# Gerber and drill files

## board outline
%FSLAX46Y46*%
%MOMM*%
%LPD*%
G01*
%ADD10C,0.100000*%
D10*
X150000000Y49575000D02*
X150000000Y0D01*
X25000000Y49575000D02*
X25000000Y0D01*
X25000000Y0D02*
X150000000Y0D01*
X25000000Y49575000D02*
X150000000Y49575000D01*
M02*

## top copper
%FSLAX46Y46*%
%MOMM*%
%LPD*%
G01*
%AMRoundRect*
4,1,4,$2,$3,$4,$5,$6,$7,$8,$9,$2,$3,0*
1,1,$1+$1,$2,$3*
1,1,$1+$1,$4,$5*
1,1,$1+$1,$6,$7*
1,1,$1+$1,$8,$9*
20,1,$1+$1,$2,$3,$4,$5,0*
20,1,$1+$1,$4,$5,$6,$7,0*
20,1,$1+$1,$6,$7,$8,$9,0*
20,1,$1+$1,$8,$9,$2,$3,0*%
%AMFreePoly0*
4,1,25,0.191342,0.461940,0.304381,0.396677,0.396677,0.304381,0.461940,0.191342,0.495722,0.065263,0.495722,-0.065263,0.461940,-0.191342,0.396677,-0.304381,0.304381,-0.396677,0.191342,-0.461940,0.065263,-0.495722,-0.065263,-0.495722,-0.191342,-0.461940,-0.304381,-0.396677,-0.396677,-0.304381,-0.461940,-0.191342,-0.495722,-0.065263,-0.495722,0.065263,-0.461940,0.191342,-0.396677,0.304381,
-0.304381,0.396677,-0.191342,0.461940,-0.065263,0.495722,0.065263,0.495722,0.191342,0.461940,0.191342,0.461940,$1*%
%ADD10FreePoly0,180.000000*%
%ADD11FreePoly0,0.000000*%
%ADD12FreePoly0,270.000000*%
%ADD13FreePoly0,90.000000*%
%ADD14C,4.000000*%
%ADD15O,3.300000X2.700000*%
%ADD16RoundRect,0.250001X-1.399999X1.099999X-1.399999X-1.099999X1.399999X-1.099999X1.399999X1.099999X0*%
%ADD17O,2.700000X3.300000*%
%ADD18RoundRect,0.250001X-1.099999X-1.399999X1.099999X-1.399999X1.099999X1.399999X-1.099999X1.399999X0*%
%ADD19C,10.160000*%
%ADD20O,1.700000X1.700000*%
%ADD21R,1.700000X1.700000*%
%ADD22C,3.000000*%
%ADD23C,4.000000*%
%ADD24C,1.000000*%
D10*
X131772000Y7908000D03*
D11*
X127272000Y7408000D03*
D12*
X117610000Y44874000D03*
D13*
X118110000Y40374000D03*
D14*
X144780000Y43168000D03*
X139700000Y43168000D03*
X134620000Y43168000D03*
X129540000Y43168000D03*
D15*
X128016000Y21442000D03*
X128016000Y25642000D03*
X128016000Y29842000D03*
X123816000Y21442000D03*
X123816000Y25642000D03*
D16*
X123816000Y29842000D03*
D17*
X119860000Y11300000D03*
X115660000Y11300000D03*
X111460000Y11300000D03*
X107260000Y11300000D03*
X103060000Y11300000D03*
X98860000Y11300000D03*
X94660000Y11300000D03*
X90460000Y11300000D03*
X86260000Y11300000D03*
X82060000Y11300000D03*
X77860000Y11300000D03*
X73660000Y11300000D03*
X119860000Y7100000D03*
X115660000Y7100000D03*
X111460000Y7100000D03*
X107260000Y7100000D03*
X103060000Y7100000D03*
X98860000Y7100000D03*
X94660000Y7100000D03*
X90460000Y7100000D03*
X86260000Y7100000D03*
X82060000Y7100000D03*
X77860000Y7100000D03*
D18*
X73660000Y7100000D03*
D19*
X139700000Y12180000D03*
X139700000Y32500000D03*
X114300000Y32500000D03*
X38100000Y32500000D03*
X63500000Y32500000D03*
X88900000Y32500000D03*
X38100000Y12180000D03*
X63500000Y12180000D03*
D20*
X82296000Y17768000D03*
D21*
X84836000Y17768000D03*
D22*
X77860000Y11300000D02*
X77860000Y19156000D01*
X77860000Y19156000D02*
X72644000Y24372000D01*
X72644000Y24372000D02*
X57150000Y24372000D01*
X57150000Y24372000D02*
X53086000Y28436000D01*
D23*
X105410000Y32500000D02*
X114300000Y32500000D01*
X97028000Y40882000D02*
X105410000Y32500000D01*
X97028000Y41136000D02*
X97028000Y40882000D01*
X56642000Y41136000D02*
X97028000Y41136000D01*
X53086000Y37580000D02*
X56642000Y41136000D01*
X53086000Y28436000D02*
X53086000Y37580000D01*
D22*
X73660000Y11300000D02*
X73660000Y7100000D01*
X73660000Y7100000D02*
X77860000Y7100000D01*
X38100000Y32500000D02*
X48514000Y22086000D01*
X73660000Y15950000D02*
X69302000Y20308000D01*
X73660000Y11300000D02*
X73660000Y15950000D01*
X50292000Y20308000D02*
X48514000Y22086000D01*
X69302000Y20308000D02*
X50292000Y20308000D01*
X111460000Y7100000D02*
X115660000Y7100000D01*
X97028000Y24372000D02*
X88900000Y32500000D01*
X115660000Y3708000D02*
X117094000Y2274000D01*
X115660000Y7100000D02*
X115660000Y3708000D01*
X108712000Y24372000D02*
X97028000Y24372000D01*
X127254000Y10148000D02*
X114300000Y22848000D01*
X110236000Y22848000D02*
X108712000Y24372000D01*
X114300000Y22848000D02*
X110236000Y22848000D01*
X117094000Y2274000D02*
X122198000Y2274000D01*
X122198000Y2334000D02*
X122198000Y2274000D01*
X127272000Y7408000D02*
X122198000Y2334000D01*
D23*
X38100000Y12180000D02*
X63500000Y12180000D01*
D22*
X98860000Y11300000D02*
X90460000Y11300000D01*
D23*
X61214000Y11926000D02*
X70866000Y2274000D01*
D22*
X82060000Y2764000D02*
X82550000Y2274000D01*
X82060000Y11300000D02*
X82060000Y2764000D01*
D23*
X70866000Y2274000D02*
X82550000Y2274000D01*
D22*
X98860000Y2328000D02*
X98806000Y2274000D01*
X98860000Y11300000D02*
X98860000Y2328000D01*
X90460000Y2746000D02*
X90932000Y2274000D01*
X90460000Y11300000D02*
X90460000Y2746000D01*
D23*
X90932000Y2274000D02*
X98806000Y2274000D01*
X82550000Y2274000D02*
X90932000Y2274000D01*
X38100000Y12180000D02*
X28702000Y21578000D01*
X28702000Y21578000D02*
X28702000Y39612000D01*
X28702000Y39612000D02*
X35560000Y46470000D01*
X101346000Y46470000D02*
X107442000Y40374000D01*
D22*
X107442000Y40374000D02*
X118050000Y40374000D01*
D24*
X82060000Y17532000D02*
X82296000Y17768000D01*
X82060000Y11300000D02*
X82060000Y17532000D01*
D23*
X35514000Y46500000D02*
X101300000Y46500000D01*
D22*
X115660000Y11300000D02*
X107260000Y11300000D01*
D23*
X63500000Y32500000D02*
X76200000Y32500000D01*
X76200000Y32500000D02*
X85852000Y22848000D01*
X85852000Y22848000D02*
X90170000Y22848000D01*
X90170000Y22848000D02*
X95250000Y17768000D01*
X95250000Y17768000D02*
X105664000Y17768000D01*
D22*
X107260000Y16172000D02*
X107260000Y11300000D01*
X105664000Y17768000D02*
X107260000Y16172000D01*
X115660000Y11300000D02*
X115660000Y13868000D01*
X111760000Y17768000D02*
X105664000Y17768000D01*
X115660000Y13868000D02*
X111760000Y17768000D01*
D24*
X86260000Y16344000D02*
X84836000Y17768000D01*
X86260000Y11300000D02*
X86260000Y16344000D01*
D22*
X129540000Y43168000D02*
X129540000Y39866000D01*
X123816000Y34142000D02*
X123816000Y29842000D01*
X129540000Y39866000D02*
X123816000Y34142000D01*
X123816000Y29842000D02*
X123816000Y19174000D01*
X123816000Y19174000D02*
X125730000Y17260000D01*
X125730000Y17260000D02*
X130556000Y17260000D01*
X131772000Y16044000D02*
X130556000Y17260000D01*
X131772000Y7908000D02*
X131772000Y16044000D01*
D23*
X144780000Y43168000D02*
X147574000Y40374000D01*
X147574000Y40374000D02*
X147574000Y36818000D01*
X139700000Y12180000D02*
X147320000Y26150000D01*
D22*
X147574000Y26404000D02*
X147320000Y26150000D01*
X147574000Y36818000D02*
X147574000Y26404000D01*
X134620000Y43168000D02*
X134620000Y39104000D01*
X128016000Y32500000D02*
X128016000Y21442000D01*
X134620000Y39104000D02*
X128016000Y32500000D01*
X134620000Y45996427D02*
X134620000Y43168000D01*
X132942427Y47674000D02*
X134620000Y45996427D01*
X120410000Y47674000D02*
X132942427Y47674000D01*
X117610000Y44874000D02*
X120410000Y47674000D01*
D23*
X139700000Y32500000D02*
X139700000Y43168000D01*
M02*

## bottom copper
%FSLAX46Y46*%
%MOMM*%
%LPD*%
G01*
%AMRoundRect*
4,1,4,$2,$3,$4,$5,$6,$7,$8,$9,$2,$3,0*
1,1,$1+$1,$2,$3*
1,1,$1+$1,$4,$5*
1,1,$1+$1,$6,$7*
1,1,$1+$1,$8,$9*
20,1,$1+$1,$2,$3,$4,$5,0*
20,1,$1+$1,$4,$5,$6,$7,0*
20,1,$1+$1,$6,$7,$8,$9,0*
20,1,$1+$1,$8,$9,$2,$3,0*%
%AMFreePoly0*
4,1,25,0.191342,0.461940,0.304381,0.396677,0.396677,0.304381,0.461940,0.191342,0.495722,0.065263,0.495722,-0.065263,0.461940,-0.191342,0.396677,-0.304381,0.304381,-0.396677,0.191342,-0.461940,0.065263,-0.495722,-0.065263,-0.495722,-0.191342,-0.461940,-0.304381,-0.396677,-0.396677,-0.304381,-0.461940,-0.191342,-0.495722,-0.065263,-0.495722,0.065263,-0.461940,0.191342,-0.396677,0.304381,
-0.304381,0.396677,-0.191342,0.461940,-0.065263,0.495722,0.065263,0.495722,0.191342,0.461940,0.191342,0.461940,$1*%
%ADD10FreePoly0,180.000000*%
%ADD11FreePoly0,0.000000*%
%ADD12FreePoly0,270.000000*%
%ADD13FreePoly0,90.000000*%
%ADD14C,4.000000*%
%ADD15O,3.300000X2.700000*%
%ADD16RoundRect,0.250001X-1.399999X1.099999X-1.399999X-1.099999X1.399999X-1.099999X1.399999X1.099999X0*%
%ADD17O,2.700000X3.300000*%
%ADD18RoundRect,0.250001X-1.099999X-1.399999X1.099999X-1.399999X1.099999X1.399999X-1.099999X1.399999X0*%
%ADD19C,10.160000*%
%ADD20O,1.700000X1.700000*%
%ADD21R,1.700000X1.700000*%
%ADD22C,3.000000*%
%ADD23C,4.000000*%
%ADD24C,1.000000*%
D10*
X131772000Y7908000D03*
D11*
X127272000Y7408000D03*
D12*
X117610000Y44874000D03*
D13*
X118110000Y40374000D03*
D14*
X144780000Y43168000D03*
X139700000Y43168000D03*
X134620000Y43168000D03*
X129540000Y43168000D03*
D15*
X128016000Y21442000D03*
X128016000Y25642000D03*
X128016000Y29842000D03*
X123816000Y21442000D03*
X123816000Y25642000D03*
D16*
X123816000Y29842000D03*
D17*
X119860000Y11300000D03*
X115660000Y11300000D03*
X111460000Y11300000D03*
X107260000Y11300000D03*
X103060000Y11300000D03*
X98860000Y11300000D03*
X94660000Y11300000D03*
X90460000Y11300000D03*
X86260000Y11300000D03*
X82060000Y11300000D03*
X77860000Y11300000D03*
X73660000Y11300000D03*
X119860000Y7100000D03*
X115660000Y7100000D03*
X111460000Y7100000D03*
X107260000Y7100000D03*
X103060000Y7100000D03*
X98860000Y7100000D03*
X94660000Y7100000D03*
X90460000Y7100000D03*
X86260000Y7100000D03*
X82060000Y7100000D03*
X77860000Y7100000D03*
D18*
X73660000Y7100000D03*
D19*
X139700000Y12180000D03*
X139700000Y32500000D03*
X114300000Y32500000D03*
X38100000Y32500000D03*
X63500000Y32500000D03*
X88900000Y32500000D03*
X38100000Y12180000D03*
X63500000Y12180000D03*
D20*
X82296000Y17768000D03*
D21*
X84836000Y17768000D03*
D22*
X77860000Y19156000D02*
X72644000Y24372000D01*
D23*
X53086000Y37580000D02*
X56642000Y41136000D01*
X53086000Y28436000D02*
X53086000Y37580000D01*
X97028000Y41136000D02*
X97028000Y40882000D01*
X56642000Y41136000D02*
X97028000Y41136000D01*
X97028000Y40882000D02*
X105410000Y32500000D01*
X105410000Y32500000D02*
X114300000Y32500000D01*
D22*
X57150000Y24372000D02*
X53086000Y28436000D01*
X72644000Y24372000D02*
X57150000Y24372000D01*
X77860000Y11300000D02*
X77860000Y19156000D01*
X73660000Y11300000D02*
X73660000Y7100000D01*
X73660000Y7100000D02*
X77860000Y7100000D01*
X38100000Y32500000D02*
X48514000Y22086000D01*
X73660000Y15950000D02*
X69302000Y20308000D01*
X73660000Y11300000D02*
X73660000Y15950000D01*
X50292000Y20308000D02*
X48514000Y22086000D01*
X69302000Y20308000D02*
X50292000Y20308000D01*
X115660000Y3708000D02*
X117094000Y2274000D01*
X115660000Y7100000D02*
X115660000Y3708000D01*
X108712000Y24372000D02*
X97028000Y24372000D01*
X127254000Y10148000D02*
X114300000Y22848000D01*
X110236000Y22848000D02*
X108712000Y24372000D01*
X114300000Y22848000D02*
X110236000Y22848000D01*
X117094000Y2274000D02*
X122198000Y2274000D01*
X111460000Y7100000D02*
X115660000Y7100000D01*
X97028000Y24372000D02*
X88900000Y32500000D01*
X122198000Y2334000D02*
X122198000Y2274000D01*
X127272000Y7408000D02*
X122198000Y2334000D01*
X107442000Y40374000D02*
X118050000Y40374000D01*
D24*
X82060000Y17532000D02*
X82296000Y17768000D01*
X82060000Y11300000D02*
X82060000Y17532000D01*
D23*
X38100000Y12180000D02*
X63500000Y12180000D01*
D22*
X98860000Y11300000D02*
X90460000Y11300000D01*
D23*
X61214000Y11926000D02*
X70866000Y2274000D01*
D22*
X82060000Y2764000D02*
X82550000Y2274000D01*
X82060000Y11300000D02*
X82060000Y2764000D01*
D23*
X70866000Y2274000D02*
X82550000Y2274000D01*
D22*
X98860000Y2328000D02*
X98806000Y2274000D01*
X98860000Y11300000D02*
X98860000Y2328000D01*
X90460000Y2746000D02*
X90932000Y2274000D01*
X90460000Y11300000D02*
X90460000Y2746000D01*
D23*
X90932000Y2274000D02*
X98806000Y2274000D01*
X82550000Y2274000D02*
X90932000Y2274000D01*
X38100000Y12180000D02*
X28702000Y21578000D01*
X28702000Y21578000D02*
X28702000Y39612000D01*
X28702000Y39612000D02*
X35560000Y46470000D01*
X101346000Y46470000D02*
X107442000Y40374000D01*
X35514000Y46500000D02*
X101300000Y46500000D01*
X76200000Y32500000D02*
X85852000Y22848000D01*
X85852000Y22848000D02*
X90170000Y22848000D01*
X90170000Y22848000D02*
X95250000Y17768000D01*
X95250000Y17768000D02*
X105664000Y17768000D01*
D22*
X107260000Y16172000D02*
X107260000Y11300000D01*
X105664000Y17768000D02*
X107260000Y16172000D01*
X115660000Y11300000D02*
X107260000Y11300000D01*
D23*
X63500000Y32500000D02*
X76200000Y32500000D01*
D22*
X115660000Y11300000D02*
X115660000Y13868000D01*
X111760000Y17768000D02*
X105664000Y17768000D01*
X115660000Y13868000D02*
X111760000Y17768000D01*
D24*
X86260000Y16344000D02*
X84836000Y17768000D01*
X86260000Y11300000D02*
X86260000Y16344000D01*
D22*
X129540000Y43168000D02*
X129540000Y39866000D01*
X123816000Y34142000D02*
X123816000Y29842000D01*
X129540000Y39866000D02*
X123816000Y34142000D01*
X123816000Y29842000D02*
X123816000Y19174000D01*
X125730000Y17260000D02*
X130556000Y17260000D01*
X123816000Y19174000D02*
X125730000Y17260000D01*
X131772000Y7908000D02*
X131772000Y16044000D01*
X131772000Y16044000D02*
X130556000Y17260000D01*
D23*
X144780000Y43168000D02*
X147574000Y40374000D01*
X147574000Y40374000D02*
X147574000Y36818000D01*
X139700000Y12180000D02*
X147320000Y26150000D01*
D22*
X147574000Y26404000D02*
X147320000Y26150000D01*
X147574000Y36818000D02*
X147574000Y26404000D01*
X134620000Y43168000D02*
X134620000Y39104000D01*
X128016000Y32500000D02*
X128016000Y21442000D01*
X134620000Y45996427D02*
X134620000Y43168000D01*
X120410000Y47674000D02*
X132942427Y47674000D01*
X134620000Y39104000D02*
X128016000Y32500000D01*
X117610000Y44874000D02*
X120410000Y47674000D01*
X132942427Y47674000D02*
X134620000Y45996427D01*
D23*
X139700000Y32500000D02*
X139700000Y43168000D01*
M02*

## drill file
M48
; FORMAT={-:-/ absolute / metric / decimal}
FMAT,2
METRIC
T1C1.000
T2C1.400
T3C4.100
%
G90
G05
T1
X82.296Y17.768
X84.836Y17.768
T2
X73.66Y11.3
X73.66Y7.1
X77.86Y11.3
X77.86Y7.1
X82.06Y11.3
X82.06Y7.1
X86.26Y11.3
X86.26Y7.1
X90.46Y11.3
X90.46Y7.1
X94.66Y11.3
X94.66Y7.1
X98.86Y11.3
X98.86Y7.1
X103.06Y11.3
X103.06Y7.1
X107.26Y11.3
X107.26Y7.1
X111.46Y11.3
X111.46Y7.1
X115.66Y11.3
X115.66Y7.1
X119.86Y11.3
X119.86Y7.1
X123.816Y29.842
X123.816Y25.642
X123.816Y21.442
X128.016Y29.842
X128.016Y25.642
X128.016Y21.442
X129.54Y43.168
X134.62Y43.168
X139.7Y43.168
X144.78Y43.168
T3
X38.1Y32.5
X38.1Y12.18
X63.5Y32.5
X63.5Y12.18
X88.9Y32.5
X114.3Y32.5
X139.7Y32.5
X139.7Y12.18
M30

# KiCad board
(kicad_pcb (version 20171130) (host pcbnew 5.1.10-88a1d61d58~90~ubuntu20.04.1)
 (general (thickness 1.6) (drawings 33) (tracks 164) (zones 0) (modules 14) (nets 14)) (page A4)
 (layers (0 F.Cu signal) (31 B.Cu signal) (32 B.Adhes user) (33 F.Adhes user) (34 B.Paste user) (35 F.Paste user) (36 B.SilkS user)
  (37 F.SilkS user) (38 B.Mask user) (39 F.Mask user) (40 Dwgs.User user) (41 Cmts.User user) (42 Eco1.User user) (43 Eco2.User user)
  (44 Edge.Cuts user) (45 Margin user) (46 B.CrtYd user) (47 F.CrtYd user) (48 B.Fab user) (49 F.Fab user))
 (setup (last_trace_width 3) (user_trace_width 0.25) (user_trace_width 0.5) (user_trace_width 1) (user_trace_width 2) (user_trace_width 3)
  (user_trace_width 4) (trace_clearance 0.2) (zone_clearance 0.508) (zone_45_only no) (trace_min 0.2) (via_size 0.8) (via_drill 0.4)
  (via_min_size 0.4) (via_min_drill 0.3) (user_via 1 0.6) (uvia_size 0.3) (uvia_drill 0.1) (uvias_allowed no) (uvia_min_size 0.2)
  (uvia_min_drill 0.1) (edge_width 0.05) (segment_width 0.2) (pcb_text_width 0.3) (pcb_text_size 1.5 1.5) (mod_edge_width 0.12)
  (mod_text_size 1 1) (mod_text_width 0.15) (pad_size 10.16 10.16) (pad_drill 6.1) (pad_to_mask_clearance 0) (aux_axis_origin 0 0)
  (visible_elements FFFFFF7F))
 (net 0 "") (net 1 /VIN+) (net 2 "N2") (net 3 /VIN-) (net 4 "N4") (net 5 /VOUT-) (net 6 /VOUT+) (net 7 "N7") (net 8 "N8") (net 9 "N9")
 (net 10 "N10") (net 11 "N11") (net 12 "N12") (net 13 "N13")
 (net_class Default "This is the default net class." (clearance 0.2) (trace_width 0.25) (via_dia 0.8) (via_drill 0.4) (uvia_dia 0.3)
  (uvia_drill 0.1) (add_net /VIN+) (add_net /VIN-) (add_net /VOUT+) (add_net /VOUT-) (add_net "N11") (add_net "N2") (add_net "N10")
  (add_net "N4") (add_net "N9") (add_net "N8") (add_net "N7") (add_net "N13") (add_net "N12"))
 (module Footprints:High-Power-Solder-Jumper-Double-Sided (layer F.Cu) (at 127.272 -7.408)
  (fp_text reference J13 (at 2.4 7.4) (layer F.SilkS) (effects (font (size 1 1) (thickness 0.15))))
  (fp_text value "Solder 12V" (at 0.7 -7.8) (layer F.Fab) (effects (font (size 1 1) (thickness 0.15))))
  (pad 2 smd custom (at 4.5 -0.5 180) (size 1 1) (layers B.Cu B.Paste B.Mask) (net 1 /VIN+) (zone_connect 0)
   (options (clearance outline) (anchor circle)) (primitives))
  (pad 1 smd custom (at 0 0) (size 1 1) (layers B.Cu B.Paste B.Mask) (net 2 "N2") (zone_connect 0)
   (options (clearance outline) (anchor circle)) (primitives))
  (pad 2 smd custom (at 4.5 -0.5 180) (size 1 1) (layers F.Cu F.Paste F.Mask) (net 1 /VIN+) (zone_connect 0)
   (options (clearance outline) (anchor circle)) (primitives))
  (pad 1 smd custom (at 0 0) (size 1 1) (layers F.Cu F.Paste F.Mask) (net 2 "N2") (zone_connect 0)
   (options (clearance outline) (anchor circle)) (primitives)))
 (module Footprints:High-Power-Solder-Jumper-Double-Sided (layer F.Cu) (at 118.11 -40.374 90)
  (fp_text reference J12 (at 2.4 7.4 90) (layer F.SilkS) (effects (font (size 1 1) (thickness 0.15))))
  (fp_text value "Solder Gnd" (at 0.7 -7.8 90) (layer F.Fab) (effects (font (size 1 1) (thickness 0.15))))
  (pad 2 smd custom (at 4.5 -0.5 270) (size 1 1) (layers B.Cu B.Paste B.Mask) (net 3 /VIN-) (zone_connect 0)
   (options (clearance outline) (anchor circle)) (primitives))
  (pad 1 smd custom (at 0 0 90) (size 1 1) (layers B.Cu B.Paste B.Mask) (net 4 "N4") (zone_connect 0)
   (options (clearance outline) (anchor circle)) (primitives))
  (pad 2 smd custom (at 4.5 -0.5 270) (size 1 1) (layers F.Cu F.Paste F.Mask) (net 3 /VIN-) (zone_connect 0)
   (options (clearance outline) (anchor circle)) (primitives))
  (pad 1 smd custom (at 0 0 90) (size 1 1) (layers F.Cu F.Paste F.Mask) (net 4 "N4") (zone_connect 0)
   (options (clearance outline) (anchor circle)) (primitives)))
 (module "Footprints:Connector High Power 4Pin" (layer F.Cu) (at 129.54 -43.168)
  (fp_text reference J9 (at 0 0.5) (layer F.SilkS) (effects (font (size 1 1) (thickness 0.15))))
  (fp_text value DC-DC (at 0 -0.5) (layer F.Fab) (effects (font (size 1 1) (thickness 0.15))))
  (pad 4 thru_hole circle (at 15.24 0) (size 4 4) (drill 1.4) (layers *.Cu *.Mask) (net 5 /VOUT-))
  (pad 3 thru_hole circle (at 10.16 0) (size 4 4) (drill 1.4) (layers *.Cu *.Mask) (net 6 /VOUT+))
  (pad 2 thru_hole circle (at 5.08 0) (size 4 4) (drill 1.4) (layers *.Cu *.Mask) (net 3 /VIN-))
  (pad 1 thru_hole circle (at 0 0) (size 4 4) (drill 1.4) (layers *.Cu *.Mask) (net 1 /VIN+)))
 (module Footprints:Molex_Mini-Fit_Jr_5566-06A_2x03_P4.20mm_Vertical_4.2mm (layer B.Cu) (at 123.816 -29.842 270)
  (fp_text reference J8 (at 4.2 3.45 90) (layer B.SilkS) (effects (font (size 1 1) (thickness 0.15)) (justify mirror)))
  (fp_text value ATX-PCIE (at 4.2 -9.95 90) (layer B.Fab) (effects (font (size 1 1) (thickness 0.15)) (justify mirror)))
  (pad 6 thru_hole oval (at 8.4 -4.2 270) (size 2.7 3.3) (drill 1.4) (layers *.Cu *.Mask) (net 3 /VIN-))
  (pad 5 thru_hole oval (at 4.2 -4.2 270) (size 2.7 3.3) (drill 1.4) (layers *.Cu *.Mask) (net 3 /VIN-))
  (pad 4 thru_hole oval (at 0 -4.2 270) (size 2.7 3.3) (drill 1.4) (layers *.Cu *.Mask) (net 3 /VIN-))
  (pad 3 thru_hole oval (at 8.4 0 270) (size 2.7 3.3) (drill 1.4) (layers *.Cu *.Mask) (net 1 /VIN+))
  (pad 2 thru_hole oval (at 4.2 0 270) (size 2.7 3.3) (drill 1.4) (layers *.Cu *.Mask) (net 1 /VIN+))
  (pad 1 thru_hole roundrect (at 0 0 270) (size 2.7 3.3) (drill 1.4) (layers *.Cu *.Mask) (roundrect_rratio 0.09259296296296296)
   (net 1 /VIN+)))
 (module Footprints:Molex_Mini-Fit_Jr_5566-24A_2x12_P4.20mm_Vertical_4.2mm (layer B.Cu) (at 73.66 -7.1)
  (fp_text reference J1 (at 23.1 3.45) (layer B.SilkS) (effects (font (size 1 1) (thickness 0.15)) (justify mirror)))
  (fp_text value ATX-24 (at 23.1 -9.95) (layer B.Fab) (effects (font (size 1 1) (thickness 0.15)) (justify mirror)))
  (pad 24 thru_hole oval (at 46.2 -4.2) (size 2.7 3.3) (drill 1.4) (layers *.Cu *.Mask) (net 4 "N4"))
  (pad 23 thru_hole oval (at 42 -4.2) (size 2.7 3.3) (drill 1.4) (layers *.Cu *.Mask) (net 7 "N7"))
  (pad 22 thru_hole oval (at 37.8 -4.2) (size 2.7 3.3) (drill 1.4) (layers *.Cu *.Mask) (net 7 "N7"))
  (pad 21 thru_hole oval (at 33.6 -4.2) (size 2.7 3.3) (drill 1.4) (layers *.Cu *.Mask) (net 7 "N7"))
  (pad 20 thru_hole oval (at 29.4 -4.2) (size 2.7 3.3) (drill 1.4) (layers *.Cu *.Mask) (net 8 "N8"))
  (pad 19 thru_hole oval (at 25.2 -4.2) (size 2.7 3.3) (drill 1.4) (layers *.Cu *.Mask) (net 4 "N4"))
  (pad 18 thru_hole oval (at 21 -4.2) (size 2.7 3.3) (drill 1.4) (layers *.Cu *.Mask) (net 4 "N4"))
  (pad 17 thru_hole oval (at 16.8 -4.2) (size 2.7 3.3) (drill 1.4) (layers *.Cu *.Mask) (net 4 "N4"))
  (pad 16 thru_hole oval (at 12.6 -4.2) (size 2.7 3.3) (drill 1.4) (layers *.Cu *.Mask) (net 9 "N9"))
  (pad 15 thru_hole oval (at 8.4 -4.2) (size 2.7 3.3) (drill 1.4) (layers *.Cu *.Mask) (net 4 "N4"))
  (pad 14 thru_hole oval (at 4.2 -4.2) (size 2.7 3.3) (drill 1.4) (layers *.Cu *.Mask) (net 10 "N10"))
  (pad 13 thru_hole oval (at 0 -4.2) (size 2.7 3.3) (drill 1.4) (layers *.Cu *.Mask) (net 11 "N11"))
  (pad 12 thru_hole oval (at 46.2 0) (size 2.7 3.3) (drill 1.4) (layers *.Cu *.Mask) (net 11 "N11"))
  (pad 11 thru_hole oval (at 42 0) (size 2.7 3.3) (drill 1.4) (layers *.Cu *.Mask) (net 2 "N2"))
  (pad 10 thru_hole oval (at 37.8 0) (size 2.7 3.3) (drill 1.4) (layers *.Cu *.Mask) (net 2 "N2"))
  (pad 9 thru_hole oval (at 33.6 0) (size 2.7 3.3) (drill 1.4) (layers *.Cu *.Mask) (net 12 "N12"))
  (pad 8 thru_hole oval (at 29.4 0) (size 2.7 3.3) (drill 1.4) (layers *.Cu *.Mask) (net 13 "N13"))
  (pad 7 thru_hole oval (at 25.2 0) (size 2.7 3.3) (drill 1.4) (layers *.Cu *.Mask) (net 4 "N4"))
  (pad 6 thru_hole oval (at 21 0) (size 2.7 3.3) (drill 1.4) (layers *.Cu *.Mask) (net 7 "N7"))
  (pad 5 thru_hole oval (at 16.8 0) (size 2.7 3.3) (drill 1.4) (layers *.Cu *.Mask) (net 4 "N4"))
  (pad 4 thru_hole oval (at 12.6 0) (size 2.7 3.3) (drill 1.4) (layers *.Cu *.Mask) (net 7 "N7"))
  (pad 3 thru_hole oval (at 8.4 0) (size 2.7 3.3) (drill 1.4) (layers *.Cu *.Mask) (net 4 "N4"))
  (pad 2 thru_hole oval (at 4.2 0) (size 2.7 3.3) (drill 1.4) (layers *.Cu *.Mask) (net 11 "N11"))
  (pad 1 thru_hole roundrect (at 0 0) (size 2.7 3.3) (drill 1.4) (layers *.Cu *.Mask) (roundrect_rratio 0.09259296296296296) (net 11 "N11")))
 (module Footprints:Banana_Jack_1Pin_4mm (layer F.Cu) (at 139.7 -12.18)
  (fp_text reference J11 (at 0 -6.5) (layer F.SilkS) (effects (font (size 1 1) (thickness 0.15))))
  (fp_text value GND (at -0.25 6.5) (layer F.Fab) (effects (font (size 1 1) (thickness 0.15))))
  (pad 1 thru_hole circle (at 0 0) (size 10.16 10.16) (drill 4.1) (layers *.Cu *.Mask) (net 5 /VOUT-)))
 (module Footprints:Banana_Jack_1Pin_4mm (layer F.Cu) (at 139.7 -32.5)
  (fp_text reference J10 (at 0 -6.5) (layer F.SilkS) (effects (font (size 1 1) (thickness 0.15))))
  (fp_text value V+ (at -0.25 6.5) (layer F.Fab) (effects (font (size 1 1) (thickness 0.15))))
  (pad 1 thru_hole circle (at 0 0) (size 10.16 10.16) (drill 4.1) (layers *.Cu *.Mask) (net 6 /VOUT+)))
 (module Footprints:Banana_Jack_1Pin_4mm (layer F.Cu) (at 114.3 -32.5)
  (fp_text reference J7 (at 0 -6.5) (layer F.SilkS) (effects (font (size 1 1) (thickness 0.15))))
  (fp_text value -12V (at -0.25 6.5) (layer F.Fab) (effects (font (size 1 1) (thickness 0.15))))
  (pad 1 thru_hole circle (at 0 0) (size 10.16 10.16) (drill 4.1) (layers *.Cu *.Mask) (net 10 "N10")))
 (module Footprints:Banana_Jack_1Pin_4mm (layer F.Cu) (at 38.1 -32.5)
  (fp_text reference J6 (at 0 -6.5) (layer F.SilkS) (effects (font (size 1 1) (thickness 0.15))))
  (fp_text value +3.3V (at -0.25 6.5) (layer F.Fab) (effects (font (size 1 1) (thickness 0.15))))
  (pad 1 thru_hole circle (at 0 0) (size 10.16 10.16) (drill 4.1) (layers *.Cu *.Mask) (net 11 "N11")))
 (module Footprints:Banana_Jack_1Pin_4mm (layer F.Cu) (at 63.5 -32.5)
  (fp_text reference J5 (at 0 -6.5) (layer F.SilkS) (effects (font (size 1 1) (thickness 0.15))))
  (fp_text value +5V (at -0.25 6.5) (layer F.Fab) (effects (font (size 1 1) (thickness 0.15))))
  (pad 1 thru_hole circle (at 0 0) (size 10.16 10.16) (drill 4.1) (layers *.Cu *.Mask) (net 7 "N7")))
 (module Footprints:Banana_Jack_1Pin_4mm (layer F.Cu) (at 88.9 -32.5)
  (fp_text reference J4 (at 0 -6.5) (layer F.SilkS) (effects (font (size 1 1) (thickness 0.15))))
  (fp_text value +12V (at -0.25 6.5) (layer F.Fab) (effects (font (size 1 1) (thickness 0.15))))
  (pad 1 thru_hole circle (at 0 0) (size 10.16 10.16) (drill 4.1) (layers *.Cu *.Mask) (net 2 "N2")))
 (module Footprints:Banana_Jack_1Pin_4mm (layer F.Cu) (at 38.1 -12.18)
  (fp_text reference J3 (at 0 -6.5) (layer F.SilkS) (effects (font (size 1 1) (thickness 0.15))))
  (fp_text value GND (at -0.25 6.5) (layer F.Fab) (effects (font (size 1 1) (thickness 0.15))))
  (pad 1 thru_hole circle (at 0 0) (size 10.16 10.16) (drill 4.1) (layers *.Cu *.Mask) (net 4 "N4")))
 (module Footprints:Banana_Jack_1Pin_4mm (layer F.Cu) (at 63.5 -12.18)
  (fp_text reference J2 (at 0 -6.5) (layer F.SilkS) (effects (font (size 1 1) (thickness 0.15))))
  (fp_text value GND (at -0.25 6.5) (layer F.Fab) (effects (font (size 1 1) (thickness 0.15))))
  (pad 1 thru_hole circle (at 0 0) (size 10.16 10.16) (drill 4.1) (layers *.Cu *.Mask) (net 4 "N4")))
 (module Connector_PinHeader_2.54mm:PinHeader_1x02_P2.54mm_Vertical (layer B.Cu) (at 84.836 -17.768 90)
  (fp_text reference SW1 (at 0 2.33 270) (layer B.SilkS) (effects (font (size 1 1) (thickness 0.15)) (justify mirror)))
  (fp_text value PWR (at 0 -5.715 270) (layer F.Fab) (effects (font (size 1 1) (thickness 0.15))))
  (pad 2 thru_hole oval (at 0 -2.54 90) (size 1.7 1.7) (drill 1) (layers *.Cu *.Mask) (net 4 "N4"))
  (pad 1 thru_hole rect (at 0 0 90) (size 1.7 1.7) (drill 1) (layers *.Cu *.Mask) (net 9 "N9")))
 (gr_line (start 150 -49.575) (end 150 0) (layer Edge.Cuts) (width 0.1))
 (gr_line (start 25 -49.575) (end 25 0) (layer Edge.Cuts) (width 0.1))
 (gr_line (start 25 0) (end 150 0) (layer Edge.Cuts) (width 0.1))
 (gr_line (start 25 -49.575) (end 150 -49.575) (layer Edge.Cuts) (width 0.1))
 (segment (start 77.86 -11.3) (end 77.86 -19.156) (width 3) (layer F.Cu) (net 10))
 (segment (start 77.86 -19.156) (end 72.644 -24.372) (width 3) (layer F.Cu) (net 10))
 (segment (start 72.644 -24.372) (end 57.15 -24.372) (width 3) (layer F.Cu) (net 10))
 (segment (start 57.15 -24.372) (end 53.086 -28.436) (width 3) (layer F.Cu) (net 10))
 (segment (start 105.41 -32.5) (end 114.3 -32.5) (width 4) (layer F.Cu) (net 10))
 (segment (start 97.028 -40.882) (end 105.41 -32.5) (width 4) (layer F.Cu) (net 10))
 (segment (start 97.028 -41.136) (end 97.028 -40.882) (width 4) (layer F.Cu) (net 10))
 (segment (start 56.642 -41.136) (end 97.028 -41.136) (width 4) (layer F.Cu) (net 10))
 (segment (start 53.086 -37.58) (end 56.642 -41.136) (width 4) (layer F.Cu) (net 10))
 (segment (start 53.086 -28.436) (end 53.086 -37.58) (width 4) (layer F.Cu) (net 10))
 (segment (start 77.86 -19.156) (end 72.644 -24.372) (width 3) (layer B.Cu) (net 10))
 (segment (start 53.086 -37.58) (end 56.642 -41.136) (width 4) (layer B.Cu) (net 10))
 (segment (start 53.086 -28.436) (end 53.086 -37.58) (width 4) (layer B.Cu) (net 10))
 (segment (start 97.028 -41.136) (end 97.028 -40.882) (width 4) (layer B.Cu) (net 10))
 (segment (start 56.642 -41.136) (end 97.028 -41.136) (width 4) (layer B.Cu) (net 10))
 (segment (start 97.028 -40.882) (end 105.41 -32.5) (width 4) (layer B.Cu) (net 10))
 (segment (start 105.41 -32.5) (end 114.3 -32.5) (width 4) (layer B.Cu) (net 10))
 (segment (start 57.15 -24.372) (end 53.086 -28.436) (width 3) (layer B.Cu) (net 10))
 (segment (start 72.644 -24.372) (end 57.15 -24.372) (width 3) (layer B.Cu) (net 10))
 (segment (start 77.86 -11.3) (end 77.86 -19.156) (width 3) (layer B.Cu) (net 10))
 (segment (start 73.66 -11.3) (end 73.66 -7.1) (width 3) (layer F.Cu) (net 11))
 (segment (start 73.66 -7.1) (end 77.86 -7.1) (width 3) (layer F.Cu) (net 11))
 (segment (start 38.1 -32.5) (end 48.514 -22.086) (width 3) (layer F.Cu) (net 11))
 (segment (start 73.66 -15.95) (end 69.302 -20.308) (width 3) (layer F.Cu) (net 11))
 (segment (start 73.66 -11.3) (end 73.66 -15.95) (width 3) (layer F.Cu) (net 11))
 (segment (start 50.292 -20.308) (end 48.514 -22.086) (width 3) (layer F.Cu) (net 11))
 (segment (start 69.302 -20.308) (end 50.292 -20.308) (width 3) (layer F.Cu) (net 11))
 (segment (start 73.66 -11.3) (end 73.66 -7.1) (width 3) (layer B.Cu) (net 11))
 (segment (start 73.66 -7.1) (end 77.86 -7.1) (width 3) (layer B.Cu) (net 11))
 (segment (start 38.1 -32.5) (end 48.514 -22.086) (width 3) (layer B.Cu) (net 11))
 (segment (start 73.66 -15.95) (end 69.302 -20.308) (width 3) (layer B.Cu) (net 11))
 (segment (start 73.66 -11.3) (end 73.66 -15.95) (width 3) (layer B.Cu) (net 11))
 (segment (start 50.292 -20.308) (end 48.514 -22.086) (width 3) (layer B.Cu) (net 11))
 (segment (start 69.302 -20.308) (end 50.292 -20.308) (width 3) (layer B.Cu) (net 11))
 (segment (start 111.46 -7.1) (end 115.66 -7.1) (width 3) (layer F.Cu) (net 2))
 (segment (start 97.028 -24.372) (end 88.9 -32.5) (width 3) (layer F.Cu) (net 2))
 (segment (start 115.66 -3.708) (end 117.094 -2.274) (width 3) (layer F.Cu) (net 2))
 (segment (start 115.66 -7.1) (end 115.66 -3.708) (width 3) (layer F.Cu) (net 2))
 (segment (start 108.712 -24.372) (end 97.028 -24.372) (width 3) (layer F.Cu) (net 2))
 (segment (start 127.254 -10.148) (end 114.3 -22.848) (width 3) (layer F.Cu) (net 2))
 (segment (start 110.236 -22.848) (end 108.712 -24.372) (width 3) (layer F.Cu) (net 2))
 (segment (start 114.3 -22.848) (end 110.236 -22.848) (width 3) (layer F.Cu) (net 2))
 (segment (start 117.094 -2.274) (end 122.198 -2.274) (width 3) (layer F.Cu) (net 2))
 (segment (start 122.198 -2.334) (end 122.198 -2.274) (width 3) (layer F.Cu) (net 2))
 (segment (start 127.272 -7.408) (end 122.198 -2.334) (width 3) (layer F.Cu) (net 2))
 (segment (start 115.66 -3.708) (end 117.094 -2.274) (width 3) (layer B.Cu) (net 2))
 (segment (start 115.66 -7.1) (end 115.66 -3.708) (width 3) (layer B.Cu) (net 2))
 (segment (start 108.712 -24.372) (end 97.028 -24.372) (width 3) (layer B.Cu) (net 2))
 (segment (start 127.254 -10.148) (end 114.3 -22.848) (width 3) (layer B.Cu) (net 2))
 (segment (start 110.236 -22.848) (end 108.712 -24.372) (width 3) (layer B.Cu) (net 2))
 (segment (start 114.3 -22.848) (end 110.236 -22.848) (width 3) (layer B.Cu) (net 2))
 (segment (start 117.094 -2.274) (end 122.198 -2.274) (width 3) (layer B.Cu) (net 2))
 (segment (start 111.46 -7.1) (end 115.66 -7.1) (width 3) (layer B.Cu) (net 2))
 (segment (start 97.028 -24.372) (end 88.9 -32.5) (width 3) (layer B.Cu) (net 2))
 (segment (start 122.198 -2.334) (end 122.198 -2.274) (width 3) (layer B.Cu) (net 2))
 (segment (start 127.272 -7.408) (end 122.198 -2.334) (width 3) (layer B.Cu) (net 2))
 (segment (start 38.1 -12.18) (end 63.5 -12.18) (width 4) (layer F.Cu) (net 4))
 (segment (start 98.86 -11.3) (end 90.46 -11.3) (width 3) (layer F.Cu) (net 4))
 (segment (start 61.214 -11.926) (end 70.866 -2.274) (width 4) (layer F.Cu) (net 4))
 (segment (start 82.06 -2.764) (end 82.55 -2.274) (width 3) (layer F.Cu) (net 4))
 (segment (start 82.06 -11.3) (end 82.06 -2.764) (width 3) (layer F.Cu) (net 4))
 (segment (start 70.866 -2.274) (end 82.55 -2.274) (width 4) (layer F.Cu) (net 4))
 (segment (start 98.86 -2.328) (end 98.806 -2.274) (width 3) (layer F.Cu) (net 4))
 (segment (start 98.86 -11.3) (end 98.86 -2.328) (width 3) (layer F.Cu) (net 4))
 (segment (start 90.46 -2.746) (end 90.932 -2.274) (width 3) (layer F.Cu) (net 4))
 (segment (start 90.46 -11.3) (end 90.46 -2.746) (width 3) (layer F.Cu) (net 4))
 (segment (start 90.932 -2.274) (end 98.806 -2.274) (width 4) (layer F.Cu) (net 4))
 (segment (start 82.55 -2.274) (end 90.932 -2.274) (width 4) (layer F.Cu) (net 4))
 (segment (start 38.1 -12.18) (end 28.702 -21.578) (width 4) (layer F.Cu) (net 4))
 (segment (start 28.702 -21.578) (end 28.702 -39.612) (width 4) (layer F.Cu) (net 4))
 (segment (start 28.702 -39.612) (end 35.56 -46.47) (width 4) (layer F.Cu) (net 4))
 (segment (start 101.346 -46.47) (end 107.442 -40.374) (width 4) (layer F.Cu) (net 4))
 (segment (start 107.442 -40.374) (end 118.05 -40.374) (width 3) (layer F.Cu) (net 4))
 (segment (start 82.06 -17.532) (end 82.296 -17.768) (width 1) (layer F.Cu) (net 4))
 (segment (start 82.06 -11.3) (end 82.06 -17.532) (width 1) (layer F.Cu) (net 4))
 (segment (start 35.514 -46.5) (end 101.3 -46.5) (width 4) (layer F.Cu) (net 4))
 (segment (start 107.442 -40.374) (end 118.05 -40.374) (width 3) (layer B.Cu) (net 4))
 (segment (start 82.06 -17.532) (end 82.296 -17.768) (width 1) (layer B.Cu) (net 4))
 (segment (start 82.06 -11.3) (end 82.06 -17.532) (width 1) (layer B.Cu) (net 4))
 (segment (start 38.1 -12.18) (end 63.5 -12.18) (width 4) (layer B.Cu) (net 4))
 (segment (start 98.86 -11.3) (end 90.46 -11.3) (width 3) (layer B.Cu) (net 4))
 (segment (start 61.214 -11.926) (end 70.866 -2.274) (width 4) (layer B.Cu) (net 4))
 (segment (start 82.06 -2.764) (end 82.55 -2.274) (width 3) (layer B.Cu) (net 4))
 (segment (start 82.06 -11.3) (end 82.06 -2.764) (width 3) (layer B.Cu) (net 4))
 (segment (start 70.866 -2.274) (end 82.55 -2.274) (width 4) (layer B.Cu) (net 4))
 (segment (start 98.86 -2.328) (end 98.806 -2.274) (width 3) (layer B.Cu) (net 4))
 (segment (start 98.86 -11.3) (end 98.86 -2.328) (width 3) (layer B.Cu) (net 4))
 (segment (start 90.46 -2.746) (end 90.932 -2.274) (width 3) (layer B.Cu) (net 4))
 (segment (start 90.46 -11.3) (end 90.46 -2.746) (width 3) (layer B.Cu) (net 4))
 (segment (start 90.932 -2.274) (end 98.806 -2.274) (width 4) (layer B.Cu) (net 4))
 (segment (start 82.55 -2.274) (end 90.932 -2.274) (width 4) (layer B.Cu) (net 4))
 (segment (start 38.1 -12.18) (end 28.702 -21.578) (width 4) (layer B.Cu) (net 4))
 (segment (start 28.702 -21.578) (end 28.702 -39.612) (width 4) (layer B.Cu) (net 4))
 (segment (start 28.702 -39.612) (end 35.56 -46.47) (width 4) (layer B.Cu) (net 4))
 (segment (start 101.346 -46.47) (end 107.442 -40.374) (width 4) (layer B.Cu) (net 4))
 (segment (start 35.514 -46.5) (end 101.3 -46.5) (width 4) (layer B.Cu) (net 4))
 (segment (start 115.66 -11.3) (end 107.26 -11.3) (width 3) (layer F.Cu) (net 7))
 (segment (start 63.5 -32.5) (end 76.2 -32.5) (width 4) (layer F.Cu) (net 7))
 (segment (start 76.2 -32.5) (end 85.852 -22.848) (width 4) (layer F.Cu) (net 7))
 (segment (start 85.852 -22.848) (end 90.17 -22.848) (width 4) (layer F.Cu) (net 7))
 (segment (start 90.17 -22.848) (end 95.25 -17.768) (width 4) (layer F.Cu) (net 7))
 (segment (start 95.25 -17.768) (end 105.664 -17.768) (width 4) (layer F.Cu) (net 7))
 (segment (start 107.26 -16.172) (end 107.26 -11.3) (width 3) (layer F.Cu) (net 7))
 (segment (start 105.664 -17.768) (end 107.26 -16.172) (width 3) (layer F.Cu) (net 7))
 (segment (start 115.66 -11.3) (end 115.66 -13.868) (width 3) (layer F.Cu) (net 7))
 (segment (start 111.76 -17.768) (end 105.664 -17.768) (width 3) (layer F.Cu) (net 7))
 (segment (start 115.66 -13.868) (end 111.76 -17.768) (width 3) (layer F.Cu) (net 7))
 (segment (start 76.2 -32.5) (end 85.852 -22.848) (width 4) (layer B.Cu) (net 7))
 (segment (start 85.852 -22.848) (end 90.17 -22.848) (width 4) (layer B.Cu) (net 7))
 (segment (start 90.17 -22.848) (end 95.25 -17.768) (width 4) (layer B.Cu) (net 7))
 (segment (start 95.25 -17.768) (end 105.664 -17.768) (width 4) (layer B.Cu) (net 7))
 (segment (start 107.26 -16.172) (end 107.26 -11.3) (width 3) (layer B.Cu) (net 7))
 (segment (start 105.664 -17.768) (end 107.26 -16.172) (width 3) (layer B.Cu) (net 7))
 (segment (start 115.66 -11.3) (end 107.26 -11.3) (width 3) (layer B.Cu) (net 7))
 (segment (start 63.5 -32.5) (end 76.2 -32.5) (width 4) (layer B.Cu) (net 7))
 (segment (start 115.66 -11.3) (end 115.66 -13.868) (width 3) (layer B.Cu) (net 7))
 (segment (start 111.76 -17.768) (end 105.664 -17.768) (width 3) (layer B.Cu) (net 7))
 (segment (start 115.66 -13.868) (end 111.76 -17.768) (width 3) (layer B.Cu) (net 7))
 (segment (start 86.26 -16.344) (end 84.836 -17.768) (width 1) (layer F.Cu) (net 9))
 (segment (start 86.26 -11.3) (end 86.26 -16.344) (width 1) (layer F.Cu) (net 9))
 (segment (start 86.26 -16.344) (end 84.836 -17.768) (width 1) (layer B.Cu) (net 9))
 (segment (start 86.26 -11.3) (end 86.26 -16.344) (width 1) (layer B.Cu) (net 9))
 (segment (start 129.54 -43.168) (end 129.54 -39.866) (width 3) (layer F.Cu) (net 1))
 (segment (start 123.816 -34.142) (end 123.816 -29.842) (width 3) (layer F.Cu) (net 1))
 (segment (start 129.54 -39.866) (end 123.816 -34.142) (width 3) (layer F.Cu) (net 1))
 (segment (start 123.816 -29.842) (end 123.816 -19.174) (width 3) (layer F.Cu) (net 1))
 (segment (start 123.816 -19.174) (end 125.73 -17.26) (width 3) (layer F.Cu) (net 1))
 (segment (start 125.73 -17.26) (end 130.556 -17.26) (width 3) (layer F.Cu) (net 1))
 (segment (start 131.772 -16.044) (end 130.556 -17.26) (width 3) (layer F.Cu) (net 1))
 (segment (start 131.772 -7.908) (end 131.772 -16.044) (width 3) (layer F.Cu) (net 1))
 (segment (start 129.54 -43.168) (end 129.54 -39.866) (width 3) (layer B.Cu) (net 1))
 (segment (start 123.816 -34.142) (end 123.816 -29.842) (width 3) (layer B.Cu) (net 1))
 (segment (start 129.54 -39.866) (end 123.816 -34.142) (width 3) (layer B.Cu) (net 1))
 (segment (start 123.816 -29.842) (end 123.816 -19.174) (width 3) (layer B.Cu) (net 1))
 (segment (start 125.73 -17.26) (end 130.556 -17.26) (width 3) (layer B.Cu) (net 1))
 (segment (start 123.816 -19.174) (end 125.73 -17.26) (width 3) (layer B.Cu) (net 1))
 (segment (start 131.772 -7.908) (end 131.772 -16.044) (width 3) (layer B.Cu) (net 1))
 (segment (start 131.772 -16.044) (end 130.556 -17.26) (width 3) (layer B.Cu) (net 1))
 (segment (start 144.78 -43.168) (end 147.574 -40.374) (width 4) (layer F.Cu) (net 5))
 (segment (start 147.574 -40.374) (end 147.574 -36.818) (width 4) (layer F.Cu) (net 5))
 (segment (start 139.7 -12.18) (end 147.32 -26.15) (width 4) (layer F.Cu) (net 5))
 (segment (start 147.574 -26.404) (end 147.32 -26.15) (width 3) (layer F.Cu) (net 5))
 (segment (start 147.574 -36.818) (end 147.574 -26.404) (width 3) (layer F.Cu) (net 5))
 (segment (start 144.78 -43.168) (end 147.574 -40.374) (width 4) (layer B.Cu) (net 5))
 (segment (start 147.574 -40.374) (end 147.574 -36.818) (width 4) (layer B.Cu) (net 5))
 (segment (start 139.7 -12.18) (end 147.32 -26.15) (width 4) (layer B.Cu) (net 5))
 (segment (start 147.574 -26.404) (end 147.32 -26.15) (width 3) (layer B.Cu) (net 5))
 (segment (start 147.574 -36.818) (end 147.574 -26.404) (width 3) (layer B.Cu) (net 5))
 (segment (start 134.62 -43.168) (end 134.62 -39.104) (width 3) (layer F.Cu) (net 3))
 (segment (start 128.016 -32.5) (end 128.016 -21.442) (width 3) (layer F.Cu) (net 3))
 (segment (start 134.62 -39.104) (end 128.016 -32.5) (width 3) (layer F.Cu) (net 3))
 (segment (start 134.62 -45.996427) (end 134.62 -43.168) (width 3) (layer F.Cu) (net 3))
 (segment (start 132.942427 -47.674) (end 134.62 -45.996427) (width 3) (layer F.Cu) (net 3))
 (segment (start 120.41 -47.674) (end 132.942427 -47.674) (width 3) (layer F.Cu) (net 3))
 (segment (start 117.61 -44.874) (end 120.41 -47.674) (width 3) (layer F.Cu) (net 3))
 (segment (start 134.62 -43.168) (end 134.62 -39.104) (width 3) (layer B.Cu) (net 3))
 (segment (start 128.016 -32.5) (end 128.016 -21.442) (width 3) (layer B.Cu) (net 3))
 (segment (start 134.62 -45.996427) (end 134.62 -43.168) (width 3) (layer B.Cu) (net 3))
 (segment (start 120.41 -47.674) (end 132.942427 -47.674) (width 3) (layer B.Cu) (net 3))
 (segment (start 134.62 -39.104) (end 128.016 -32.5) (width 3) (layer B.Cu) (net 3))
 (segment (start 117.61 -44.874) (end 120.41 -47.674) (width 3) (layer B.Cu) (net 3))
 (segment (start 132.942427 -47.674) (end 134.62 -45.996427) (width 3) (layer B.Cu) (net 3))
 (segment (start 139.7 -32.5) (end 139.7 -43.168) (width 4) (layer F.Cu) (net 6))
 (segment (start 139.7 -32.5) (end 139.7 -43.168) (width 4) (layer B.Cu) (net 6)))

